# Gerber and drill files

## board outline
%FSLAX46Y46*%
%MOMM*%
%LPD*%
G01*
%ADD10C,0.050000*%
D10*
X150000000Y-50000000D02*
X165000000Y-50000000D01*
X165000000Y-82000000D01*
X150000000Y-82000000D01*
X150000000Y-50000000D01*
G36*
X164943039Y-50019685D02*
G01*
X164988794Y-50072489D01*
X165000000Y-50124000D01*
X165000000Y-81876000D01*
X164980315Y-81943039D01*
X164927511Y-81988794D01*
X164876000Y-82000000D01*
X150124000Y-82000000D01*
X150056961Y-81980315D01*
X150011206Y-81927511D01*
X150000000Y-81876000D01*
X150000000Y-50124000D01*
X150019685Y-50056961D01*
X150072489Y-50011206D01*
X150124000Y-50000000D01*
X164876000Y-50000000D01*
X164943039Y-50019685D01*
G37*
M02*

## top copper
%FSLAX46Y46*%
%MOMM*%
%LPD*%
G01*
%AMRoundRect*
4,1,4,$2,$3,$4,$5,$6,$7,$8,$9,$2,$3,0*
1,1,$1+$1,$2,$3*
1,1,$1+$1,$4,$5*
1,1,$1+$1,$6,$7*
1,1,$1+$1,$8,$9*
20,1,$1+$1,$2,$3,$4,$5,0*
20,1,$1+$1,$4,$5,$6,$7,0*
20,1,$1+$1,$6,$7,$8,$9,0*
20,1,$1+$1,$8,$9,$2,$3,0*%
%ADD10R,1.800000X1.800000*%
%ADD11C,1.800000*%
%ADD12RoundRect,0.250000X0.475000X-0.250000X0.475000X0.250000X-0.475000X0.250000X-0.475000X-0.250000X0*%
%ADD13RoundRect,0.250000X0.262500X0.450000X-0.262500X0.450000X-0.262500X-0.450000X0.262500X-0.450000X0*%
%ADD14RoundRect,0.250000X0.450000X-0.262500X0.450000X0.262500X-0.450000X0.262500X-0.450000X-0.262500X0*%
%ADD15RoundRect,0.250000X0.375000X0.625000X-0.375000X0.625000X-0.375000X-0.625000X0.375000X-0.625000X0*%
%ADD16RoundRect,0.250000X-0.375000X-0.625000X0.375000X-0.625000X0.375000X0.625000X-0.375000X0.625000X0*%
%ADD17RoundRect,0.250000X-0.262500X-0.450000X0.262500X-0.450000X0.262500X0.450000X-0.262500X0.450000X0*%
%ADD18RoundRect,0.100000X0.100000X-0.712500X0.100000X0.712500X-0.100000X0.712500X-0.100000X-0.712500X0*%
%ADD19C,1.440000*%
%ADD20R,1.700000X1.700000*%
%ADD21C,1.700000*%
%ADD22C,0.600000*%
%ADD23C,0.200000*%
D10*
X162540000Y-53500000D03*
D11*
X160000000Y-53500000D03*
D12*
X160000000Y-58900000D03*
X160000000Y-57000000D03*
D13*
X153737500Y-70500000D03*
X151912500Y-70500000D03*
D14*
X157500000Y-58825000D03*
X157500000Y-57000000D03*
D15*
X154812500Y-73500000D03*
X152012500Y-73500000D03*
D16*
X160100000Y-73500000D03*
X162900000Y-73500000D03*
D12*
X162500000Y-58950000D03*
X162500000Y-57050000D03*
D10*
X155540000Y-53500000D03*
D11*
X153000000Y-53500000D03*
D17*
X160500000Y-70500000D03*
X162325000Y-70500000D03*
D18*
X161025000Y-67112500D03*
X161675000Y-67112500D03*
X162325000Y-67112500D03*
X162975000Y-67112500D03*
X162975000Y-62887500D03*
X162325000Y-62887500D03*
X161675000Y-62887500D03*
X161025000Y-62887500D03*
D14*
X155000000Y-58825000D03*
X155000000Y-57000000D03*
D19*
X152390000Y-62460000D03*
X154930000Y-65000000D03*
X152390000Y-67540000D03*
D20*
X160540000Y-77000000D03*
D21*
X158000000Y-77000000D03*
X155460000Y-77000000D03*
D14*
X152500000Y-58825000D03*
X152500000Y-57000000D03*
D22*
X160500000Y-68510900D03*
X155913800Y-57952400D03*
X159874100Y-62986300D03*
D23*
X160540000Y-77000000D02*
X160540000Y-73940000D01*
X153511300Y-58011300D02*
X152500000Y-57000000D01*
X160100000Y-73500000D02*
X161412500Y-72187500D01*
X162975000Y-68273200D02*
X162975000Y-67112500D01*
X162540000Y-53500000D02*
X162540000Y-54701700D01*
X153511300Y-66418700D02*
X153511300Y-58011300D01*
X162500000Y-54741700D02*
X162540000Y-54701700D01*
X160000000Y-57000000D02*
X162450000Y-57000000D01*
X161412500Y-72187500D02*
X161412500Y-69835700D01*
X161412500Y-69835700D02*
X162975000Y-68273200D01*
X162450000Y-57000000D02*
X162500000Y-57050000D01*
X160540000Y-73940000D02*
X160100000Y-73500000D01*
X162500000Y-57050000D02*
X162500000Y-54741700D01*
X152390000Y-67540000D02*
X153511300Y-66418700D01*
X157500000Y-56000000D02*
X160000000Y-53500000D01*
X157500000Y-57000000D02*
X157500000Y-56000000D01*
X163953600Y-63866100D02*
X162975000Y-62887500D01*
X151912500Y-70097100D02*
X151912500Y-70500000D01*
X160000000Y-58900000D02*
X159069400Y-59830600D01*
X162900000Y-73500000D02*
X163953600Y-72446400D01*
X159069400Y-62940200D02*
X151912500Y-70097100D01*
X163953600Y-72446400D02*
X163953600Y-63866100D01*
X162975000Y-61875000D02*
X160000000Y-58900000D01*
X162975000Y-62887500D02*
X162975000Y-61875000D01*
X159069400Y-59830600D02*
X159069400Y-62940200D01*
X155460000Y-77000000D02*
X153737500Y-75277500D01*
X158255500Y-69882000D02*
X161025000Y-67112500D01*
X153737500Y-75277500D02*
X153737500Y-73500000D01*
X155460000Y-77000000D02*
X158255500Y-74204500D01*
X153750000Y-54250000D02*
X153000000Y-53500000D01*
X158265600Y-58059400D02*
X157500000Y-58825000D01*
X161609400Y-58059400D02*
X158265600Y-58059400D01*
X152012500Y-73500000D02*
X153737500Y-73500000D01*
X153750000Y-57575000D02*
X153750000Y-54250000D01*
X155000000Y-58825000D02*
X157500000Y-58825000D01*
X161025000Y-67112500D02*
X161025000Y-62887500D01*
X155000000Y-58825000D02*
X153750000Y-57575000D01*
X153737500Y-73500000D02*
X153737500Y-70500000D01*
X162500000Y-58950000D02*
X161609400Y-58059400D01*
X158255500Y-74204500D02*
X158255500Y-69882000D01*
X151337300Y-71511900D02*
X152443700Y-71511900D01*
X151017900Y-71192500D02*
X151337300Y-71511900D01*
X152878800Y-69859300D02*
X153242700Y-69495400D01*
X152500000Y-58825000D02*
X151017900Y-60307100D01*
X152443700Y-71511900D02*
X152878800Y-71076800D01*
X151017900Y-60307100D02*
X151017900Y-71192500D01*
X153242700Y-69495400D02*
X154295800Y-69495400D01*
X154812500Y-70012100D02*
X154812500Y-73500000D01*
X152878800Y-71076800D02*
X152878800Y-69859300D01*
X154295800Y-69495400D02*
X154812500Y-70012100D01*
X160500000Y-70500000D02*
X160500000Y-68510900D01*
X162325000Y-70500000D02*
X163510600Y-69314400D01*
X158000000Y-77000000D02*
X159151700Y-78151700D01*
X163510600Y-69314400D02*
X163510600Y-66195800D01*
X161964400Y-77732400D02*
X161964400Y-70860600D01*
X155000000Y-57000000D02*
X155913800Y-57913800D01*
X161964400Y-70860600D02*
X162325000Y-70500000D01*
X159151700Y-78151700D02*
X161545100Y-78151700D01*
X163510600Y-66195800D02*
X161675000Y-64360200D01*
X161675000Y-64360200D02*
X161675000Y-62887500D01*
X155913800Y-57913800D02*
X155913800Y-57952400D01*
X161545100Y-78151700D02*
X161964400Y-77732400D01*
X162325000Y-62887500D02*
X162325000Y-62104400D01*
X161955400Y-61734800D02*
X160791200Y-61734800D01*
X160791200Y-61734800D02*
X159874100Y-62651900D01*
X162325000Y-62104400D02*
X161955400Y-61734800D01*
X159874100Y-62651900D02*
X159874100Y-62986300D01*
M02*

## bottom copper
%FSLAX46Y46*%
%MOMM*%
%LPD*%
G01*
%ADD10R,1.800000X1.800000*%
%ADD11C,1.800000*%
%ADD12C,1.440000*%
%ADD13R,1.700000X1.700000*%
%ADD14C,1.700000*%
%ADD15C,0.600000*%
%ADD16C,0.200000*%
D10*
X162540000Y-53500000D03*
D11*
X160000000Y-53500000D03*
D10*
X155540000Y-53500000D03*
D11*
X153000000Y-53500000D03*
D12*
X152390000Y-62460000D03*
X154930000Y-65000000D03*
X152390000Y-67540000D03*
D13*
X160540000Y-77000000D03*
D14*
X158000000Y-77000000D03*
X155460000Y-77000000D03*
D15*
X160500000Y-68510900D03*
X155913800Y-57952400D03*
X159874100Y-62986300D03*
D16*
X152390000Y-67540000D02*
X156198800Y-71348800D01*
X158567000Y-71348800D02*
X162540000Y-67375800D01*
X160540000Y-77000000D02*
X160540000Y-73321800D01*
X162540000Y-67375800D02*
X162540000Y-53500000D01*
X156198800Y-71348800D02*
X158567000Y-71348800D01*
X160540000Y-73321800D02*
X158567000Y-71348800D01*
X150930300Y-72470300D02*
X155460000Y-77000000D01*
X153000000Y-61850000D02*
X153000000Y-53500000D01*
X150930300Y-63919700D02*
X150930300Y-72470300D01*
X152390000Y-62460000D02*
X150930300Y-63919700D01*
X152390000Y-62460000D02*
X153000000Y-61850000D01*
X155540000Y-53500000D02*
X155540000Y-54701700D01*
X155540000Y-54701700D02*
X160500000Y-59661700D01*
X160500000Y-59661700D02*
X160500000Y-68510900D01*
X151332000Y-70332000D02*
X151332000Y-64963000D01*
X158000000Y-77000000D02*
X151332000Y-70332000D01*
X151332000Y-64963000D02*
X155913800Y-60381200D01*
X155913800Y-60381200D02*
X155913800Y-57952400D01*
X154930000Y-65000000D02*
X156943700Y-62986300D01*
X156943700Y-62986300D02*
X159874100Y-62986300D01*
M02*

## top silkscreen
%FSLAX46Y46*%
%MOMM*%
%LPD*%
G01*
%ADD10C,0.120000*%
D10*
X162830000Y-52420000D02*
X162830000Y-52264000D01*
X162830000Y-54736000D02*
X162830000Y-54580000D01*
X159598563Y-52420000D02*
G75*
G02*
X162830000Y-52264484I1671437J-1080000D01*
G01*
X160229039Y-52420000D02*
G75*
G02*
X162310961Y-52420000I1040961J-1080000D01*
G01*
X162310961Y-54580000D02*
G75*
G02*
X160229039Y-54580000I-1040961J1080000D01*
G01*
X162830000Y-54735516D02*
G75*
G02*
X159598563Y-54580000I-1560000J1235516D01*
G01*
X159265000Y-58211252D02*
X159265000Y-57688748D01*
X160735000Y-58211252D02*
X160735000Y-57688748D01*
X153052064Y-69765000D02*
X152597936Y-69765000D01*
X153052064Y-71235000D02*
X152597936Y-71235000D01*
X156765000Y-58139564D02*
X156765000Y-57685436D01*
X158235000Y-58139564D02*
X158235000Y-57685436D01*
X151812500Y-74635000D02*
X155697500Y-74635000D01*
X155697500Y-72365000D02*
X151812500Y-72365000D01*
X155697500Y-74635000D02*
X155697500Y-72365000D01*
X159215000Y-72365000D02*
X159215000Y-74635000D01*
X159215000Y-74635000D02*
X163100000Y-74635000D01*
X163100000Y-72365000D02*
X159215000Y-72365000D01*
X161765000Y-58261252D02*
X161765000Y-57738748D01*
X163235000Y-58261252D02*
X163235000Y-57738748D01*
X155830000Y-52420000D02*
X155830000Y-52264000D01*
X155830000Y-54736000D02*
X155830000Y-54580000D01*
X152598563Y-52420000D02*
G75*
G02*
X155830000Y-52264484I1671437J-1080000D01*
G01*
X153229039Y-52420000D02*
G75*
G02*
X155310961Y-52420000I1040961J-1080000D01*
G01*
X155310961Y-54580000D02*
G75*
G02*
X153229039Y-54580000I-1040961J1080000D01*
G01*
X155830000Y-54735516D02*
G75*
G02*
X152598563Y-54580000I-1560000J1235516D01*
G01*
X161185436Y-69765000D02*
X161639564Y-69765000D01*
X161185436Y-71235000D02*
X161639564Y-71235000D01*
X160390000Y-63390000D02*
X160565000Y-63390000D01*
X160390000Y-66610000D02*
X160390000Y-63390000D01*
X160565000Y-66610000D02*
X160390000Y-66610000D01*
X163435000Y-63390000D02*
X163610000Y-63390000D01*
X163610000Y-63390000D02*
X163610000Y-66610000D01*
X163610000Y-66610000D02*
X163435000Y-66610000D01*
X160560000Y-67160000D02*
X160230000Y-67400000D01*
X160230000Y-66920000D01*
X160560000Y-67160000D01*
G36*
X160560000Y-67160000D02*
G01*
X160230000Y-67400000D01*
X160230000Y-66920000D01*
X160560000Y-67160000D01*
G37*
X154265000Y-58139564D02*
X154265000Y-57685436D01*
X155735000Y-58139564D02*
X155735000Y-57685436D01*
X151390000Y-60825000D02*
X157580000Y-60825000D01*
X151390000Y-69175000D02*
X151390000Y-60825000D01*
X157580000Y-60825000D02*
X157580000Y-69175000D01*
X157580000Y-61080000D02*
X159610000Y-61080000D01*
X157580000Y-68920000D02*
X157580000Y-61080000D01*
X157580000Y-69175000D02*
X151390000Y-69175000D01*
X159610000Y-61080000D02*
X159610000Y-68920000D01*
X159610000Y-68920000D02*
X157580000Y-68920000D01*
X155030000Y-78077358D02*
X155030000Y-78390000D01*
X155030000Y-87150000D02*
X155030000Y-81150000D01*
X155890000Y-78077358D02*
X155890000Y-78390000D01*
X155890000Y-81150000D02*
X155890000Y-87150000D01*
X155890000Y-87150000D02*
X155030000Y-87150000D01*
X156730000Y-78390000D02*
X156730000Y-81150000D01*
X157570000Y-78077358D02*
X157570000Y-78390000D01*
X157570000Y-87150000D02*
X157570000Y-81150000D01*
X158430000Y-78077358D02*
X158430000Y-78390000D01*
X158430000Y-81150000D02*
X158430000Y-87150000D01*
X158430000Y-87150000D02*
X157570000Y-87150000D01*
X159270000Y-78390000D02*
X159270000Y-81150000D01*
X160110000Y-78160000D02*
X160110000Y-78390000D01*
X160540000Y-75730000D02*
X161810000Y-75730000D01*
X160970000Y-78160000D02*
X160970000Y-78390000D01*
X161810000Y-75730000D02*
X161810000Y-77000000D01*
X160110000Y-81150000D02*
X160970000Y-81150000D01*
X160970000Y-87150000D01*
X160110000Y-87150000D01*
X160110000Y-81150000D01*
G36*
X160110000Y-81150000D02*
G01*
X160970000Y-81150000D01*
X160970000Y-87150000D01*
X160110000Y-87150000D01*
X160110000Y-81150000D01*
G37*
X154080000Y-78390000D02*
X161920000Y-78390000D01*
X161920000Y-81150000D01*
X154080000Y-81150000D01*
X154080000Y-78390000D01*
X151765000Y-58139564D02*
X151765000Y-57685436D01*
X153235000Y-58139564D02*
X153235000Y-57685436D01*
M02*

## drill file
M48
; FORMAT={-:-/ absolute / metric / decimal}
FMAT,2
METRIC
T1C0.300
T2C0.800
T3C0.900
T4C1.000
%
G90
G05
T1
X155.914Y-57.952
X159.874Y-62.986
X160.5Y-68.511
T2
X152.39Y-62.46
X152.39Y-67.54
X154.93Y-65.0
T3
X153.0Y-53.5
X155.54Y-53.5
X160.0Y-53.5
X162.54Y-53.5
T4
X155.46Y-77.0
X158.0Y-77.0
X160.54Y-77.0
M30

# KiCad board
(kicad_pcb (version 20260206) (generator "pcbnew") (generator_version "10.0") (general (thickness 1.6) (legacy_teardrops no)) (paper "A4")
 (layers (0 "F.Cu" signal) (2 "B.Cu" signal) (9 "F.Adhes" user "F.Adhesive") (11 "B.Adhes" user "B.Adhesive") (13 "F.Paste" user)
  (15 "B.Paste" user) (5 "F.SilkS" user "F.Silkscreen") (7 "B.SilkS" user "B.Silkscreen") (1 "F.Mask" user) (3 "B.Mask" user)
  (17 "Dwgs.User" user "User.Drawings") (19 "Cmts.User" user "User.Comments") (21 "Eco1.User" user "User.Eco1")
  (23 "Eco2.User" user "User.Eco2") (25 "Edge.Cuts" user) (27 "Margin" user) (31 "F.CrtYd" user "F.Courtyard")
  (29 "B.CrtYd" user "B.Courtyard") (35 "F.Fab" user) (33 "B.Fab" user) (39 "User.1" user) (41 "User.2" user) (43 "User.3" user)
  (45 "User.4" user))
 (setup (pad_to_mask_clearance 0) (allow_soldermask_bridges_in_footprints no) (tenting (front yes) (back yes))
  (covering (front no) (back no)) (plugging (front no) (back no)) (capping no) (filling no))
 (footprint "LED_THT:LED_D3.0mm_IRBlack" (layer "F.Cu") (at 162.54 53.5 180)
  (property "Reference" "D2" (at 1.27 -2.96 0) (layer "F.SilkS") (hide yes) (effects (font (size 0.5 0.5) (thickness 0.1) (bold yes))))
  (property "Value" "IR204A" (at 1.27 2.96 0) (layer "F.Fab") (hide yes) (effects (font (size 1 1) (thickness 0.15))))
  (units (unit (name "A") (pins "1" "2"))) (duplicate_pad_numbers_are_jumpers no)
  (fp_line (start -0.29 1.08) (end -0.29 1.236) (stroke (width 0.12) (type solid)) (layer "F.SilkS"))
  (fp_line (start -0.29 -1.236) (end -0.29 -1.08) (stroke (width 0.12) (type solid)) (layer "F.SilkS"))
  (fp_arc (start 2.941437 1.08) (mid 1.36566 1.987699) (end -0.29 1.235516) (stroke (width 0.12) (type solid)) (layer "F.SilkS"))
  (fp_arc (start 2.310961 1.08) (mid 1.27 1.5) (end 0.229039 1.08) (stroke (width 0.12) (type solid)) (layer "F.SilkS"))
  (fp_arc (start 0.229039 -1.08) (mid 1.27 -1.5) (end 2.310961 -1.08) (stroke (width 0.12) (type solid)) (layer "F.SilkS"))
  (fp_arc (start -0.29 -1.235516) (mid 1.36566 -1.987699) (end 2.941437 -1.08) (stroke (width 0.12) (type solid)) (layer "F.SilkS"))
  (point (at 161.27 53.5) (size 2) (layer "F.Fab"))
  (pad "1" thru_hole rect (at 0 0 180) (size 1.8 1.8) (drill 0.9) (layers "*.Cu" "*.Mask") (remove_unused_layers no) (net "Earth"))
  (pad "2" thru_hole circle (at 2.54 0 180) (size 1.8 1.8) (drill 0.9) (layers "*.Cu" "*.Mask") (remove_unused_layers no) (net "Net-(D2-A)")))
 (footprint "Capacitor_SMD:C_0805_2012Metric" (layer "F.Cu") (at 160 57.95 90)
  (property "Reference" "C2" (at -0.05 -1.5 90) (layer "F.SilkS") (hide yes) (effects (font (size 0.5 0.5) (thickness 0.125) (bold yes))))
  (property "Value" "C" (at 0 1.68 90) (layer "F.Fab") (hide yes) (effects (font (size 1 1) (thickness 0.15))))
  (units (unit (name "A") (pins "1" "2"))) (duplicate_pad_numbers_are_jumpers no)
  (fp_line (start -0.261252 -0.735) (end 0.261252 -0.735) (stroke (width 0.12) (type solid)) (layer "F.SilkS"))
  (fp_line (start -0.261252 0.735) (end 0.261252 0.735) (stroke (width 0.12) (type solid)) (layer "F.SilkS"))
  (pad "1" smd roundrect (at -0.95 0 90) (size 1 1.45) (layers "F.Cu" "F.Mask" "F.Paste") (roundrect_rratio 0.25) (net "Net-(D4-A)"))
  (pad "2" smd roundrect (at 0.95 0 90) (size 1 1.45) (layers "F.Cu" "F.Mask" "F.Paste") (roundrect_rratio 0.25) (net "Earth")))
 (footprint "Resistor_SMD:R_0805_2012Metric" (layer "F.Cu") (at 152.825 70.5 180)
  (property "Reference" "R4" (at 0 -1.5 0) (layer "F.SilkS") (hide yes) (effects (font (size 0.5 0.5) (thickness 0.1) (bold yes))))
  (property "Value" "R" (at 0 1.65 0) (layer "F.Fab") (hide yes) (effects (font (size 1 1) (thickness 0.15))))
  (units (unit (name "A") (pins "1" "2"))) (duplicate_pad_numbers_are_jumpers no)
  (fp_line (start -0.227064 0.735) (end 0.227064 0.735) (stroke (width 0.12) (type solid)) (layer "F.SilkS"))
  (fp_line (start -0.227064 -0.735) (end 0.227064 -0.735) (stroke (width 0.12) (type solid)) (layer "F.SilkS"))
  (pad "1" smd roundrect (at -0.9125 0 180) (size 1.025 1.4) (layers "F.Cu" "F.Mask" "F.Paste") (roundrect_rratio 0.243902) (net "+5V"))
  (pad "2" smd roundrect (at 0.9125 0 180) (size 1.025 1.4) (layers "F.Cu" "F.Mask" "F.Paste") (roundrect_rratio 0.243902)
   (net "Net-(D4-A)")))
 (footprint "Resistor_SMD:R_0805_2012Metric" (layer "F.Cu") (at 157.5 57.9125 90)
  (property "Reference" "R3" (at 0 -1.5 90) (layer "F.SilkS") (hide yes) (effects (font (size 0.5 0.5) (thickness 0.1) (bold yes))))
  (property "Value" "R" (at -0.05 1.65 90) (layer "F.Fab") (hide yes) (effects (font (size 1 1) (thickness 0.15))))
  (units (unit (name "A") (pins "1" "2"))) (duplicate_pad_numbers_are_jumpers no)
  (fp_line (start -0.227064 -0.735) (end 0.227064 -0.735) (stroke (width 0.12) (type solid)) (layer "F.SilkS"))
  (fp_line (start -0.227064 0.735) (end 0.227064 0.735) (stroke (width 0.12) (type solid)) (layer "F.SilkS"))
  (pad "1" smd roundrect (at -0.9125 0 90) (size 1.025 1.4) (layers "F.Cu" "F.Mask" "F.Paste") (roundrect_rratio 0.243902) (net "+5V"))
  (pad "2" smd roundrect (at 0.9125 0 90) (size 1.025 1.4) (layers "F.Cu" "F.Mask" "F.Paste") (roundrect_rratio 0.243902) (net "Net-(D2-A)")))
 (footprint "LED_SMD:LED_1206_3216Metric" (layer "F.Cu") (at 153.4125 73.5 180)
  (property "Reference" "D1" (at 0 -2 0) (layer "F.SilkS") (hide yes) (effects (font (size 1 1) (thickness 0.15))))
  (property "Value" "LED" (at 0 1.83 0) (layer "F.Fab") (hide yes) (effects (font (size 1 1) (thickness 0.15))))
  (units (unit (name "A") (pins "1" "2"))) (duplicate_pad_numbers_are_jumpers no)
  (fp_line (start 1.6 -1.135) (end -2.285 -1.135) (stroke (width 0.12) (type solid)) (layer "F.SilkS"))
  (fp_line (start -2.285 1.135) (end 1.6 1.135) (stroke (width 0.12) (type solid)) (layer "F.SilkS"))
  (fp_line (start -2.285 -1.135) (end -2.285 1.135) (stroke (width 0.12) (type solid)) (layer "F.SilkS"))
  (pad "1" smd roundrect (at -1.4 0 180) (size 1.25 1.75) (layers "F.Cu" "F.Mask" "F.Paste") (roundrect_rratio 0.2) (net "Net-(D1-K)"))
  (pad "2" smd roundrect (at 1.4 0 180) (size 1.25 1.75) (layers "F.Cu" "F.Mask" "F.Paste") (roundrect_rratio 0.2) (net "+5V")))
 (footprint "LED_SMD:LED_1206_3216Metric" (layer "F.Cu") (at 161.5 73.5)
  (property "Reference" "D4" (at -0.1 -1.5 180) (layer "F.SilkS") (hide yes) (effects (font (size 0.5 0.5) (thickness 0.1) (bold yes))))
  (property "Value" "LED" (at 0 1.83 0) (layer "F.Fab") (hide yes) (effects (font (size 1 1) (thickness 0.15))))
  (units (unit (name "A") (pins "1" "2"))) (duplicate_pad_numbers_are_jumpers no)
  (fp_line (start -2.285 -1.135) (end -2.285 1.135) (stroke (width 0.12) (type solid)) (layer "F.SilkS"))
  (fp_line (start -2.285 1.135) (end 1.6 1.135) (stroke (width 0.12) (type solid)) (layer "F.SilkS"))
  (fp_line (start 1.6 -1.135) (end -2.285 -1.135) (stroke (width 0.12) (type solid)) (layer "F.SilkS"))
  (pad "1" smd roundrect (at -1.4 0) (size 1.25 1.75) (layers "F.Cu" "F.Mask" "F.Paste") (roundrect_rratio 0.2) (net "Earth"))
  (pad "2" smd roundrect (at 1.4 0) (size 1.25 1.75) (layers "F.Cu" "F.Mask" "F.Paste") (roundrect_rratio 0.2) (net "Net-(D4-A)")))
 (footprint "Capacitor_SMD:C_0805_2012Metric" (layer "F.Cu") (at 162.5 58 90)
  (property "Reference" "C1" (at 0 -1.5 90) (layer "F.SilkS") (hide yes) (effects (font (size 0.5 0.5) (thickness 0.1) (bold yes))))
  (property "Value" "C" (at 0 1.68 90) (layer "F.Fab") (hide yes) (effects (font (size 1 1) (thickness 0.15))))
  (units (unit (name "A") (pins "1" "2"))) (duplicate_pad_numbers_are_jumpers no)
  (fp_line (start -0.261252 -0.735) (end 0.261252 -0.735) (stroke (width 0.12) (type solid)) (layer "F.SilkS"))
  (fp_line (start -0.261252 0.735) (end 0.261252 0.735) (stroke (width 0.12) (type solid)) (layer "F.SilkS"))
  (pad "1" smd roundrect (at -0.95 0 90) (size 1 1.45) (layers "F.Cu" "F.Mask" "F.Paste") (roundrect_rratio 0.25) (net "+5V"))
  (pad "2" smd roundrect (at 0.95 0 90) (size 1 1.45) (layers "F.Cu" "F.Mask" "F.Paste") (roundrect_rratio 0.25) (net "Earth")))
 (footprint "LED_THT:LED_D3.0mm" (layer "F.Cu") (at 155.54 53.5 180)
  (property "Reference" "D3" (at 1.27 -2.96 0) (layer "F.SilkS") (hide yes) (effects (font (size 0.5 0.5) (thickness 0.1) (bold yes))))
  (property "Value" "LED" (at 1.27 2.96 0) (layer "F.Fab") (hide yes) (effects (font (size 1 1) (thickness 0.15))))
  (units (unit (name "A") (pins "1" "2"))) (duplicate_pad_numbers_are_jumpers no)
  (fp_line (start -0.29 1.08) (end -0.29 1.236) (stroke (width 0.12) (type solid)) (layer "F.SilkS"))
  (fp_line (start -0.29 -1.236) (end -0.29 -1.08) (stroke (width 0.12) (type solid)) (layer "F.SilkS"))
  (fp_arc (start 2.941437 1.08) (mid 1.36566 1.987699) (end -0.29 1.235516) (stroke (width 0.12) (type solid)) (layer "F.SilkS"))
  (fp_arc (start 2.310961 1.08) (mid 1.27 1.5) (end 0.229039 1.08) (stroke (width 0.12) (type solid)) (layer "F.SilkS"))
  (fp_arc (start 0.229039 -1.08) (mid 1.27 -1.5) (end 2.310961 -1.08) (stroke (width 0.12) (type solid)) (layer "F.SilkS"))
  (fp_arc (start -0.29 -1.235516) (mid 1.36566 -1.987699) (end 2.941437 -1.08) (stroke (width 0.12) (type solid)) (layer "F.SilkS"))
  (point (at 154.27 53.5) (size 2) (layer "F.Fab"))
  (pad "1" thru_hole rect (at 0 0 180) (size 1.8 1.8) (drill 0.9) (layers "*.Cu" "*.Mask") (remove_unused_layers no) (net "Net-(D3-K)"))
  (pad "2" thru_hole circle (at 2.54 0 180) (size 1.8 1.8) (drill 0.9) (layers "*.Cu" "*.Mask") (remove_unused_layers no) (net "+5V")))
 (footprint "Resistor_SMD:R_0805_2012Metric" (layer "F.Cu") (at 161.4125 70.5)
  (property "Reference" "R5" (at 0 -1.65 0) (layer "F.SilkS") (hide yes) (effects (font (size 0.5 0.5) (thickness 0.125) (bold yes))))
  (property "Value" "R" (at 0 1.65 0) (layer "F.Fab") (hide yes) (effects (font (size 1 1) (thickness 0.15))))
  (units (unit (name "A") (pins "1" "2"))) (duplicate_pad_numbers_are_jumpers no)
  (fp_line (start -0.227064 -0.735) (end 0.227064 -0.735) (stroke (width 0.12) (type solid)) (layer "F.SilkS"))
  (fp_line (start -0.227064 0.735) (end 0.227064 0.735) (stroke (width 0.12) (type solid)) (layer "F.SilkS"))
  (pad "1" smd roundrect (at -0.9125 0) (size 1.025 1.4) (layers "F.Cu" "F.Mask" "F.Paste") (roundrect_rratio 0.243902) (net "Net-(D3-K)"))
  (pad "2" smd roundrect (at 0.9125 0) (size 1.025 1.4) (layers "F.Cu" "F.Mask" "F.Paste") (roundrect_rratio 0.243902)
   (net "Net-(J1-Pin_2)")))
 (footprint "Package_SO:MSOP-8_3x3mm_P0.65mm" (layer "F.Cu") (at 162 65 90)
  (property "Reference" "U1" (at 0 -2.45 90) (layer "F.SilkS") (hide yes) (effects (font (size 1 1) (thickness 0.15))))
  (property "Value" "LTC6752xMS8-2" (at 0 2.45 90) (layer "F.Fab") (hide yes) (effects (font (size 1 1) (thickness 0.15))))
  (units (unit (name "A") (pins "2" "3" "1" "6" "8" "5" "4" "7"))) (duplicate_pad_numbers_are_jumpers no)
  (fp_line (start 1.61 -1.61) (end 1.61 -1.435) (stroke (width 0.12) (type solid)) (layer "F.SilkS"))
  (fp_line (start -1.61 -1.61) (end 1.61 -1.61) (stroke (width 0.12) (type solid)) (layer "F.SilkS"))
  (fp_line (start -1.61 -1.435) (end -1.61 -1.61) (stroke (width 0.12) (type solid)) (layer "F.SilkS"))
  (fp_line (start 1.61 1.435) (end 1.61 1.61) (stroke (width 0.12) (type solid)) (layer "F.SilkS"))
  (fp_line (start 1.61 1.61) (end -1.61 1.61) (stroke (width 0.12) (type solid)) (layer "F.SilkS"))
  (fp_line (start -1.61 1.61) (end -1.61 1.435) (stroke (width 0.12) (type solid)) (layer "F.SilkS"))
  (fp_poly (pts (xy -2.16 -1.44) (xy -2.4 -1.77) (xy -1.92 -1.77)) (stroke (width 0.12) (type solid)) (fill yes) (layer "F.SilkS"))
  (pad "1" smd roundrect (at -2.1125 -0.975 90) (size 1.625 0.4) (layers "F.Cu" "F.Mask" "F.Paste") (roundrect_rratio 0.25) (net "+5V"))
  (pad "2" smd roundrect (at -2.1125 -0.325 90) (size 1.625 0.4) (layers "F.Cu" "F.Mask" "F.Paste") (roundrect_rratio 0.25)
   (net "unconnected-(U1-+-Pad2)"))
  (pad "3" smd roundrect (at -2.1125 0.325 90) (size 1.625 0.4) (layers "F.Cu" "F.Mask" "F.Paste") (roundrect_rratio 0.25)
   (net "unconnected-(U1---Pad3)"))
  (pad "4" smd roundrect (at -2.1125 0.975 90) (size 1.625 0.4) (layers "F.Cu" "F.Mask" "F.Paste") (roundrect_rratio 0.25) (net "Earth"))
  (pad "5" smd roundrect (at 2.1125 0.975 90) (size 1.625 0.4) (layers "F.Cu" "F.Mask" "F.Paste") (roundrect_rratio 0.25) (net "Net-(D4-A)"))
  (pad "6" smd roundrect (at 2.1125 0.325 90) (size 1.625 0.4) (layers "F.Cu" "F.Mask" "F.Paste") (roundrect_rratio 0.25)
   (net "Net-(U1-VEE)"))
  (pad "7" smd roundrect (at 2.1125 -0.325 90) (size 1.625 0.4) (layers "F.Cu" "F.Mask" "F.Paste") (roundrect_rratio 0.25)
   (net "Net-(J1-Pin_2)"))
  (pad "8" smd roundrect (at 2.1125 -0.975 90) (size 1.625 0.4) (layers "F.Cu" "F.Mask" "F.Paste") (roundrect_rratio 0.25) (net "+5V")))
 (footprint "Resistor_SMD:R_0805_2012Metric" (layer "F.Cu") (at 155 57.9125 90)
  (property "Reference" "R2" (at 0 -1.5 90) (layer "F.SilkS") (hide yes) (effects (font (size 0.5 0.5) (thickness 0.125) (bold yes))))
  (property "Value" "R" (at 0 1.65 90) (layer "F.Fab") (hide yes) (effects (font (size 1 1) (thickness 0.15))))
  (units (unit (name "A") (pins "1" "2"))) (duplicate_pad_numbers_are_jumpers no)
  (fp_line (start -0.227064 -0.735) (end 0.227064 -0.735) (stroke (width 0.12) (type solid)) (layer "F.SilkS"))
  (fp_line (start -0.227064 0.735) (end 0.227064 0.735) (stroke (width 0.12) (type solid)) (layer "F.SilkS"))
  (pad "1" smd roundrect (at -0.9125 0 90) (size 1.025 1.4) (layers "F.Cu" "F.Mask" "F.Paste") (roundrect_rratio 0.243902) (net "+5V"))
  (pad "2" smd roundrect (at 0.9125 0 90) (size 1.025 1.4) (layers "F.Cu" "F.Mask" "F.Paste") (roundrect_rratio 0.243902)
   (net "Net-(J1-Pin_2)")))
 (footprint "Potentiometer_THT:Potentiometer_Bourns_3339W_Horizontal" (layer "F.Cu") (at 152.39 62.46)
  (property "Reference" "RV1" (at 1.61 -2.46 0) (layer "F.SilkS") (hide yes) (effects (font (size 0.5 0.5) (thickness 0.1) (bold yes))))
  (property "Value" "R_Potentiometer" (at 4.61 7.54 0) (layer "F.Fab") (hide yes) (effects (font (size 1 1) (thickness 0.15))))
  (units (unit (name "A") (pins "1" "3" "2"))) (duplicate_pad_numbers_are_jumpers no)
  (fp_line (start -1 -1.635) (end 5.19 -1.635) (stroke (width 0.12) (type solid)) (layer "F.SilkS"))
  (fp_line (start -1 6.715) (end -1 -1.635) (stroke (width 0.12) (type solid)) (layer "F.SilkS"))
  (fp_line (start 5.19 -1.635) (end 5.19 6.715) (stroke (width 0.12) (type solid)) (layer "F.SilkS"))
  (fp_line (start 5.19 -1.38) (end 7.22 -1.38) (stroke (width 0.12) (type solid)) (layer "F.SilkS"))
  (fp_line (start 5.19 6.46) (end 5.19 -1.38) (stroke (width 0.12) (type solid)) (layer "F.SilkS"))
  (fp_line (start 5.19 6.715) (end -1 6.715) (stroke (width 0.12) (type solid)) (layer "F.SilkS"))
  (fp_line (start 7.22 -1.38) (end 7.22 6.46) (stroke (width 0.12) (type solid)) (layer "F.SilkS"))
  (fp_line (start 7.22 6.46) (end 5.19 6.46) (stroke (width 0.12) (type solid)) (layer "F.SilkS"))
  (pad "1" thru_hole circle (at 0 0) (size 1.44 1.44) (drill 0.8) (layers "*.Cu" "*.Mask") (remove_unused_layers no) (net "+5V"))
  (pad "2" thru_hole circle (at 2.54 2.54) (size 1.44 1.44) (drill 0.8) (layers "*.Cu" "*.Mask") (remove_unused_layers no)
   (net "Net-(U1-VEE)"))
  (pad "3" thru_hole circle (at 0 5.08) (size 1.44 1.44) (drill 0.8) (layers "*.Cu" "*.Mask") (remove_unused_layers no) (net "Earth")))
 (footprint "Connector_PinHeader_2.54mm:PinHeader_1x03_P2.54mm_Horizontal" (layer "F.Cu") (at 160.54 77 -90)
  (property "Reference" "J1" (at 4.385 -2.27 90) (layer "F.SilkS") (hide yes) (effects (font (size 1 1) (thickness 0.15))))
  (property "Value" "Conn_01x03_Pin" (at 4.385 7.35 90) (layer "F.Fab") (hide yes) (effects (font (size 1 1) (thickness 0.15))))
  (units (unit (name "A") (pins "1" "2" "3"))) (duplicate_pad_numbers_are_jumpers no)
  (fp_line (start 1.077358 5.51) (end 1.39 5.51) (stroke (width 0.12) (type solid)) (layer "F.SilkS"))
  (fp_line (start 10.15 5.51) (end 4.15 5.51) (stroke (width 0.12) (type solid)) (layer "F.SilkS"))
  (fp_line (start 1.077358 4.65) (end 1.39 4.65) (stroke (width 0.12) (type solid)) (layer "F.SilkS"))
  (fp_line (start 4.15 4.65) (end 10.15 4.65) (stroke (width 0.12) (type solid)) (layer "F.SilkS"))
  (fp_line (start 10.15 4.65) (end 10.15 5.51) (stroke (width 0.12) (type solid)) (layer "F.SilkS"))
  (fp_line (start 1.39 3.81) (end 4.15 3.81) (stroke (width 0.12) (type solid)) (layer "F.SilkS"))
  (fp_line (start 1.077358 2.97) (end 1.39 2.97) (stroke (width 0.12) (type solid)) (layer "F.SilkS"))
  (fp_line (start 10.15 2.97) (end 4.15 2.97) (stroke (width 0.12) (type solid)) (layer "F.SilkS"))
  (fp_line (start 1.077358 2.11) (end 1.39 2.11) (stroke (width 0.12) (type solid)) (layer "F.SilkS"))
  (fp_line (start 4.15 2.11) (end 10.15 2.11) (stroke (width 0.12) (type solid)) (layer "F.SilkS"))
  (fp_line (start 10.15 2.11) (end 10.15 2.97) (stroke (width 0.12) (type solid)) (layer "F.SilkS"))
  (fp_line (start 1.39 1.27) (end 4.15 1.27) (stroke (width 0.12) (type solid)) (layer "F.SilkS"))
  (fp_line (start 1.16 0.43) (end 1.39 0.43) (stroke (width 0.12) (type solid)) (layer "F.SilkS"))
  (fp_line (start -1.27 0) (end -1.27 -1.27) (stroke (width 0.12) (type solid)) (layer "F.SilkS"))
  (fp_line (start 1.16 -0.43) (end 1.39 -0.43) (stroke (width 0.12) (type solid)) (layer "F.SilkS"))
  (fp_line (start -1.27 -1.27) (end 0 -1.27) (stroke (width 0.12) (type solid)) (layer "F.SilkS"))
  (fp_rect (start 4.15 -0.43) (end 10.15 0.43) (stroke (width 0.12) (type solid)) (fill yes) (layer "F.SilkS"))
  (fp_rect (start 1.39 -1.38) (end 4.15 6.46) (stroke (width 0.12) (type solid)) (fill no) (layer "F.SilkS"))
  (pad "1" thru_hole rect (at 0 0 270) (size 1.7 1.7) (drill 1) (layers "*.Cu" "*.Mask") (remove_unused_layers no) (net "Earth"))
  (pad "2" thru_hole circle (at 0 2.54 270) (size 1.7 1.7) (drill 1) (layers "*.Cu" "*.Mask") (remove_unused_layers no)
   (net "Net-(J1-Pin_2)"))
  (pad "3" thru_hole circle (at 0 5.08 270) (size 1.7 1.7) (drill 1) (layers "*.Cu" "*.Mask") (remove_unused_layers no) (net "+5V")))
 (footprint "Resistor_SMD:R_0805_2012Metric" (layer "F.Cu") (at 152.5 57.9125 90)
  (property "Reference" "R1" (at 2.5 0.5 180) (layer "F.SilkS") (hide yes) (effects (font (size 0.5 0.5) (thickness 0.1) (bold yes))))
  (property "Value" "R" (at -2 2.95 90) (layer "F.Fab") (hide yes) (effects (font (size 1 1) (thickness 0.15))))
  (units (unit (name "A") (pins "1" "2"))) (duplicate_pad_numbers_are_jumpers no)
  (fp_line (start -0.227064 -0.735) (end 0.227064 -0.735) (stroke (width 0.12) (type solid)) (layer "F.SilkS"))
  (fp_line (start -0.227064 0.735) (end 0.227064 0.735) (stroke (width 0.12) (type solid)) (layer "F.SilkS"))
  (pad "1" smd roundrect (at -0.9125 0 90) (size 1.025 1.4) (layers "F.Cu" "F.Mask" "F.Paste") (roundrect_rratio 0.243902)
   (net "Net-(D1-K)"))
  (pad "2" smd roundrect (at 0.9125 0 90) (size 1.025 1.4) (layers "F.Cu" "F.Mask" "F.Paste") (roundrect_rratio 0.243902) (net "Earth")))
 (gr_rect (start 150 50) (end 165 82) (stroke (width 0.05) (type default)) (fill no) (layer "Edge.Cuts"))
 (segment (start 160.54 77) (end 160.54 73.94) (width 0.2) (layer "F.Cu") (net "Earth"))
 (segment (start 153.5113 58.0113) (end 152.5 57) (width 0.2) (layer "F.Cu") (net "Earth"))
 (segment (start 160.1 73.5) (end 161.4125 72.1875) (width 0.2) (layer "F.Cu") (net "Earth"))
 (segment (start 162.975 68.2732) (end 162.975 67.1125) (width 0.2) (layer "F.Cu") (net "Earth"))
 (segment (start 162.54 53.5) (end 162.54 54.7017) (width 0.2) (layer "F.Cu") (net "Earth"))
 (segment (start 153.5113 66.4187) (end 153.5113 58.0113) (width 0.2) (layer "F.Cu") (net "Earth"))
 (segment (start 162.5 54.7417) (end 162.54 54.7017) (width 0.2) (layer "F.Cu") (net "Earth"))
 (segment (start 160 57) (end 162.45 57) (width 0.2) (layer "F.Cu") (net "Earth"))
 (segment (start 161.4125 72.1875) (end 161.4125 69.8357) (width 0.2) (layer "F.Cu") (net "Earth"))
 (segment (start 161.4125 69.8357) (end 162.975 68.2732) (width 0.2) (layer "F.Cu") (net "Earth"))
 (segment (start 162.45 57) (end 162.5 57.05) (width 0.2) (layer "F.Cu") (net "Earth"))
 (segment (start 160.54 73.94) (end 160.1 73.5) (width 0.2) (layer "F.Cu") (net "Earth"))
 (segment (start 162.5 57.05) (end 162.5 54.7417) (width 0.2) (layer "F.Cu") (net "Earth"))
 (segment (start 152.39 67.54) (end 153.5113 66.4187) (width 0.2) (layer "F.Cu") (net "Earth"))
 (segment (start 152.39 67.54) (end 156.1988 71.3488) (width 0.2) (layer "B.Cu") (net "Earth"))
 (segment (start 158.567 71.3488) (end 162.54 67.3758) (width 0.2) (layer "B.Cu") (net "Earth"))
 (segment (start 160.54 77) (end 160.54 73.3218) (width 0.2) (layer "B.Cu") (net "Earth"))
 (segment (start 162.54 67.3758) (end 162.54 53.5) (width 0.2) (layer "B.Cu") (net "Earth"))
 (segment (start 156.1988 71.3488) (end 158.567 71.3488) (width 0.2) (layer "B.Cu") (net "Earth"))
 (segment (start 160.54 73.3218) (end 158.567 71.3488) (width 0.2) (layer "B.Cu") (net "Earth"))
 (segment (start 157.5 56) (end 160 53.5) (width 0.2) (layer "F.Cu") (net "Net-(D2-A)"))
 (segment (start 157.5 57) (end 157.5 56) (width 0.2) (layer "F.Cu") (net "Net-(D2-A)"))
 (segment (start 163.9536 63.8661) (end 162.975 62.8875) (width 0.2) (layer "F.Cu") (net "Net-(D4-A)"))
 (segment (start 151.9125 70.0971) (end 151.9125 70.5) (width 0.2) (layer "F.Cu") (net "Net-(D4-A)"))
 (segment (start 160 58.9) (end 159.0694 59.8306) (width 0.2) (layer "F.Cu") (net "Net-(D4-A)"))
 (segment (start 162.9 73.5) (end 163.9536 72.4464) (width 0.2) (layer "F.Cu") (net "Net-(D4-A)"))
 (segment (start 159.0694 62.9402) (end 151.9125 70.0971) (width 0.2) (layer "F.Cu") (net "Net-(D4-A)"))
 (segment (start 163.9536 72.4464) (end 163.9536 63.8661) (width 0.2) (layer "F.Cu") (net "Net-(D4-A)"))
 (segment (start 162.975 61.875) (end 160 58.9) (width 0.2) (layer "F.Cu") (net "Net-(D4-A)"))
 (segment (start 162.975 62.8875) (end 162.975 61.875) (width 0.2) (layer "F.Cu") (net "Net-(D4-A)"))
 (segment (start 159.0694 59.8306) (end 159.0694 62.9402) (width 0.2) (layer "F.Cu") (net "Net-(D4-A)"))
 (segment (start 155.46 77) (end 153.7375 75.2775) (width 0.2) (layer "F.Cu") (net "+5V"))
 (segment (start 158.2555 69.882) (end 161.025 67.1125) (width 0.2) (layer "F.Cu") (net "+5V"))
 (segment (start 153.7375 75.2775) (end 153.7375 73.5) (width 0.2) (layer "F.Cu") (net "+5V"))
 (segment (start 155.46 77) (end 158.2555 74.2045) (width 0.2) (layer "F.Cu") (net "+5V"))
 (segment (start 153.75 54.25) (end 153 53.5) (width 0.2) (layer "F.Cu") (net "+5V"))
 (segment (start 158.2656 58.0594) (end 157.5 58.825) (width 0.2) (layer "F.Cu") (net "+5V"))
 (segment (start 161.6094 58.0594) (end 158.2656 58.0594) (width 0.2) (layer "F.Cu") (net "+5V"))
 (segment (start 152.0125 73.5) (end 153.7375 73.5) (width 0.2) (layer "F.Cu") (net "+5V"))
 (segment (start 153.75 57.575) (end 153.75 54.25) (width 0.2) (layer "F.Cu") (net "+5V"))
 (segment (start 155 58.825) (end 157.5 58.825) (width 0.2) (layer "F.Cu") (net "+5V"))
 (segment (start 161.025 67.1125) (end 161.025 62.8875) (width 0.2) (layer "F.Cu") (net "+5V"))
 (segment (start 155 58.825) (end 153.75 57.575) (width 0.2) (layer "F.Cu") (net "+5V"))
 (segment (start 153.7375 73.5) (end 153.7375 70.5) (width 0.2) (layer "F.Cu") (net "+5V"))
 (segment (start 162.5 58.95) (end 161.6094 58.0594) (width 0.2) (layer "F.Cu") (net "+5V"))
 (segment (start 158.2555 74.2045) (end 158.2555 69.882) (width 0.2) (layer "F.Cu") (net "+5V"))
 (segment (start 150.9303 72.4703) (end 155.46 77) (width 0.2) (layer "B.Cu") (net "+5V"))
 (segment (start 153 61.85) (end 153 53.5) (width 0.2) (layer "B.Cu") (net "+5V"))
 (segment (start 150.9303 63.9197) (end 150.9303 72.4703) (width 0.2) (layer "B.Cu") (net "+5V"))
 (segment (start 152.39 62.46) (end 150.9303 63.9197) (width 0.2) (layer "B.Cu") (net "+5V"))
 (segment (start 152.39 62.46) (end 153 61.85) (width 0.2) (layer "B.Cu") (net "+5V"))
 (segment (start 151.3373 71.5119) (end 152.4437 71.5119) (width 0.2) (layer "F.Cu") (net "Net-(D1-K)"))
 (segment (start 151.0179 71.1925) (end 151.3373 71.5119) (width 0.2) (layer "F.Cu") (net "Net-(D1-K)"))
 (segment (start 152.8788 69.8593) (end 153.2427 69.4954) (width 0.2) (layer "F.Cu") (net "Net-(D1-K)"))
 (segment (start 152.5 58.825) (end 151.0179 60.3071) (width 0.2) (layer "F.Cu") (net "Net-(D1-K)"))
 (segment (start 152.4437 71.5119) (end 152.8788 71.0768) (width 0.2) (layer "F.Cu") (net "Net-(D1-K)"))
 (segment (start 151.0179 60.3071) (end 151.0179 71.1925) (width 0.2) (layer "F.Cu") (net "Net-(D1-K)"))
 (segment (start 153.2427 69.4954) (end 154.2958 69.4954) (width 0.2) (layer "F.Cu") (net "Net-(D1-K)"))
 (segment (start 154.8125 70.0121) (end 154.8125 73.5) (width 0.2) (layer "F.Cu") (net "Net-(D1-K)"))
 (segment (start 152.8788 71.0768) (end 152.8788 69.8593) (width 0.2) (layer "F.Cu") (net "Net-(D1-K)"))
 (segment (start 154.2958 69.4954) (end 154.8125 70.0121) (width 0.2) (layer "F.Cu") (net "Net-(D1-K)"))
 (segment (start 160.5 70.5) (end 160.5 68.5109) (width 0.2) (layer "F.Cu") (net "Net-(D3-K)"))
 (via (at 160.5 68.5109) (size 0.6) (drill 0.3) (layers "F.Cu" "B.Cu") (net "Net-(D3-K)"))
 (segment (start 155.54 53.5) (end 155.54 54.7017) (width 0.2) (layer "B.Cu") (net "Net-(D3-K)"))
 (segment (start 155.54 54.7017) (end 160.5 59.6617) (width 0.2) (layer "B.Cu") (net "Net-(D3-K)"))
 (segment (start 160.5 59.6617) (end 160.5 68.5109) (width 0.2) (layer "B.Cu") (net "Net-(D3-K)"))
 (segment (start 162.325 70.5) (end 163.5106 69.3144) (width 0.2) (layer "F.Cu") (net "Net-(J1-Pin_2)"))
 (segment (start 158 77) (end 159.1517 78.1517) (width 0.2) (layer "F.Cu") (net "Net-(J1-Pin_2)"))
 (segment (start 163.5106 69.3144) (end 163.5106 66.1958) (width 0.2) (layer "F.Cu") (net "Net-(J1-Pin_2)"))
 (segment (start 161.9644 77.7324) (end 161.9644 70.8606) (width 0.2) (layer "F.Cu") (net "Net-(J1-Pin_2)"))
 (segment (start 155 57) (end 155.9138 57.9138) (width 0.2) (layer "F.Cu") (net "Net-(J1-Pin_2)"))
 (segment (start 161.9644 70.8606) (end 162.325 70.5) (width 0.2) (layer "F.Cu") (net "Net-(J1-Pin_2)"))
 (segment (start 159.1517 78.1517) (end 161.5451 78.1517) (width 0.2) (layer "F.Cu") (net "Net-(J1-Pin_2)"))
 (segment (start 163.5106 66.1958) (end 161.675 64.3602) (width 0.2) (layer "F.Cu") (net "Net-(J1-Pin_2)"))
 (segment (start 161.675 64.3602) (end 161.675 62.8875) (width 0.2) (layer "F.Cu") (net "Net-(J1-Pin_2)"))
 (segment (start 155.9138 57.9138) (end 155.9138 57.9524) (width 0.2) (layer "F.Cu") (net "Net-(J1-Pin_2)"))
 (segment (start 161.5451 78.1517) (end 161.9644 77.7324) (width 0.2) (layer "F.Cu") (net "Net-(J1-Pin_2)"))
 (via (at 155.9138 57.9524) (size 0.6) (drill 0.3) (layers "F.Cu" "B.Cu") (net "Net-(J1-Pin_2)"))
 (segment (start 151.332 70.332) (end 151.332 64.963) (width 0.2) (layer "B.Cu") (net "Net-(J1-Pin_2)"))
 (segment (start 158 77) (end 151.332 70.332) (width 0.2) (layer "B.Cu") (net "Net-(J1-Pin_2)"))
 (segment (start 151.332 64.963) (end 155.9138 60.3812) (width 0.2) (layer "B.Cu") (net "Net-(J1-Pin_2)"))
 (segment (start 155.9138 60.3812) (end 155.9138 57.9524) (width 0.2) (layer "B.Cu") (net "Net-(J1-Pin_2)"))
 (segment (start 162.325 62.8875) (end 162.325 62.1044) (width 0.2) (layer "F.Cu") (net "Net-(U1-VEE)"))
 (segment (start 161.9554 61.7348) (end 160.7912 61.7348) (width 0.2) (layer "F.Cu") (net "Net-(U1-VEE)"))
 (segment (start 160.7912 61.7348) (end 159.8741 62.6519) (width 0.2) (layer "F.Cu") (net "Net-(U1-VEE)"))
 (segment (start 162.325 62.1044) (end 161.9554 61.7348) (width 0.2) (layer "F.Cu") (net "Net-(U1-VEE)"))
 (segment (start 159.8741 62.6519) (end 159.8741 62.9863) (width 0.2) (layer "F.Cu") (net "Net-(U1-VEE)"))
 (via (at 159.8741 62.9863) (size 0.6) (drill 0.3) (layers "F.Cu" "B.Cu") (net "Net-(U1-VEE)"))
 (segment (start 154.93 65) (end 156.9437 62.9863) (width 0.2) (layer "B.Cu") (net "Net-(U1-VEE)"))
 (segment (start 156.9437 62.9863) (end 159.8741 62.9863) (width 0.2) (layer "B.Cu") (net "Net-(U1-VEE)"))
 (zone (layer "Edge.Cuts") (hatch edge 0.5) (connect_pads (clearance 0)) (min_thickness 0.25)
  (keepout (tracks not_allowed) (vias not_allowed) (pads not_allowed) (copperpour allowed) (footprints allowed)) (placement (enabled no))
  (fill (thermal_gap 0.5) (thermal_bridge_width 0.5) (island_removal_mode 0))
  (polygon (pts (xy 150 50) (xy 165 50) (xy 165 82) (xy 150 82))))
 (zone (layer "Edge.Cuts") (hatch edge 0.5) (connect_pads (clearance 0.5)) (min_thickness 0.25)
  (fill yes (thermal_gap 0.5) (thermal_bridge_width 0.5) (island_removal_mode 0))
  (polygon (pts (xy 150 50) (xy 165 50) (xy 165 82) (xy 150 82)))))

